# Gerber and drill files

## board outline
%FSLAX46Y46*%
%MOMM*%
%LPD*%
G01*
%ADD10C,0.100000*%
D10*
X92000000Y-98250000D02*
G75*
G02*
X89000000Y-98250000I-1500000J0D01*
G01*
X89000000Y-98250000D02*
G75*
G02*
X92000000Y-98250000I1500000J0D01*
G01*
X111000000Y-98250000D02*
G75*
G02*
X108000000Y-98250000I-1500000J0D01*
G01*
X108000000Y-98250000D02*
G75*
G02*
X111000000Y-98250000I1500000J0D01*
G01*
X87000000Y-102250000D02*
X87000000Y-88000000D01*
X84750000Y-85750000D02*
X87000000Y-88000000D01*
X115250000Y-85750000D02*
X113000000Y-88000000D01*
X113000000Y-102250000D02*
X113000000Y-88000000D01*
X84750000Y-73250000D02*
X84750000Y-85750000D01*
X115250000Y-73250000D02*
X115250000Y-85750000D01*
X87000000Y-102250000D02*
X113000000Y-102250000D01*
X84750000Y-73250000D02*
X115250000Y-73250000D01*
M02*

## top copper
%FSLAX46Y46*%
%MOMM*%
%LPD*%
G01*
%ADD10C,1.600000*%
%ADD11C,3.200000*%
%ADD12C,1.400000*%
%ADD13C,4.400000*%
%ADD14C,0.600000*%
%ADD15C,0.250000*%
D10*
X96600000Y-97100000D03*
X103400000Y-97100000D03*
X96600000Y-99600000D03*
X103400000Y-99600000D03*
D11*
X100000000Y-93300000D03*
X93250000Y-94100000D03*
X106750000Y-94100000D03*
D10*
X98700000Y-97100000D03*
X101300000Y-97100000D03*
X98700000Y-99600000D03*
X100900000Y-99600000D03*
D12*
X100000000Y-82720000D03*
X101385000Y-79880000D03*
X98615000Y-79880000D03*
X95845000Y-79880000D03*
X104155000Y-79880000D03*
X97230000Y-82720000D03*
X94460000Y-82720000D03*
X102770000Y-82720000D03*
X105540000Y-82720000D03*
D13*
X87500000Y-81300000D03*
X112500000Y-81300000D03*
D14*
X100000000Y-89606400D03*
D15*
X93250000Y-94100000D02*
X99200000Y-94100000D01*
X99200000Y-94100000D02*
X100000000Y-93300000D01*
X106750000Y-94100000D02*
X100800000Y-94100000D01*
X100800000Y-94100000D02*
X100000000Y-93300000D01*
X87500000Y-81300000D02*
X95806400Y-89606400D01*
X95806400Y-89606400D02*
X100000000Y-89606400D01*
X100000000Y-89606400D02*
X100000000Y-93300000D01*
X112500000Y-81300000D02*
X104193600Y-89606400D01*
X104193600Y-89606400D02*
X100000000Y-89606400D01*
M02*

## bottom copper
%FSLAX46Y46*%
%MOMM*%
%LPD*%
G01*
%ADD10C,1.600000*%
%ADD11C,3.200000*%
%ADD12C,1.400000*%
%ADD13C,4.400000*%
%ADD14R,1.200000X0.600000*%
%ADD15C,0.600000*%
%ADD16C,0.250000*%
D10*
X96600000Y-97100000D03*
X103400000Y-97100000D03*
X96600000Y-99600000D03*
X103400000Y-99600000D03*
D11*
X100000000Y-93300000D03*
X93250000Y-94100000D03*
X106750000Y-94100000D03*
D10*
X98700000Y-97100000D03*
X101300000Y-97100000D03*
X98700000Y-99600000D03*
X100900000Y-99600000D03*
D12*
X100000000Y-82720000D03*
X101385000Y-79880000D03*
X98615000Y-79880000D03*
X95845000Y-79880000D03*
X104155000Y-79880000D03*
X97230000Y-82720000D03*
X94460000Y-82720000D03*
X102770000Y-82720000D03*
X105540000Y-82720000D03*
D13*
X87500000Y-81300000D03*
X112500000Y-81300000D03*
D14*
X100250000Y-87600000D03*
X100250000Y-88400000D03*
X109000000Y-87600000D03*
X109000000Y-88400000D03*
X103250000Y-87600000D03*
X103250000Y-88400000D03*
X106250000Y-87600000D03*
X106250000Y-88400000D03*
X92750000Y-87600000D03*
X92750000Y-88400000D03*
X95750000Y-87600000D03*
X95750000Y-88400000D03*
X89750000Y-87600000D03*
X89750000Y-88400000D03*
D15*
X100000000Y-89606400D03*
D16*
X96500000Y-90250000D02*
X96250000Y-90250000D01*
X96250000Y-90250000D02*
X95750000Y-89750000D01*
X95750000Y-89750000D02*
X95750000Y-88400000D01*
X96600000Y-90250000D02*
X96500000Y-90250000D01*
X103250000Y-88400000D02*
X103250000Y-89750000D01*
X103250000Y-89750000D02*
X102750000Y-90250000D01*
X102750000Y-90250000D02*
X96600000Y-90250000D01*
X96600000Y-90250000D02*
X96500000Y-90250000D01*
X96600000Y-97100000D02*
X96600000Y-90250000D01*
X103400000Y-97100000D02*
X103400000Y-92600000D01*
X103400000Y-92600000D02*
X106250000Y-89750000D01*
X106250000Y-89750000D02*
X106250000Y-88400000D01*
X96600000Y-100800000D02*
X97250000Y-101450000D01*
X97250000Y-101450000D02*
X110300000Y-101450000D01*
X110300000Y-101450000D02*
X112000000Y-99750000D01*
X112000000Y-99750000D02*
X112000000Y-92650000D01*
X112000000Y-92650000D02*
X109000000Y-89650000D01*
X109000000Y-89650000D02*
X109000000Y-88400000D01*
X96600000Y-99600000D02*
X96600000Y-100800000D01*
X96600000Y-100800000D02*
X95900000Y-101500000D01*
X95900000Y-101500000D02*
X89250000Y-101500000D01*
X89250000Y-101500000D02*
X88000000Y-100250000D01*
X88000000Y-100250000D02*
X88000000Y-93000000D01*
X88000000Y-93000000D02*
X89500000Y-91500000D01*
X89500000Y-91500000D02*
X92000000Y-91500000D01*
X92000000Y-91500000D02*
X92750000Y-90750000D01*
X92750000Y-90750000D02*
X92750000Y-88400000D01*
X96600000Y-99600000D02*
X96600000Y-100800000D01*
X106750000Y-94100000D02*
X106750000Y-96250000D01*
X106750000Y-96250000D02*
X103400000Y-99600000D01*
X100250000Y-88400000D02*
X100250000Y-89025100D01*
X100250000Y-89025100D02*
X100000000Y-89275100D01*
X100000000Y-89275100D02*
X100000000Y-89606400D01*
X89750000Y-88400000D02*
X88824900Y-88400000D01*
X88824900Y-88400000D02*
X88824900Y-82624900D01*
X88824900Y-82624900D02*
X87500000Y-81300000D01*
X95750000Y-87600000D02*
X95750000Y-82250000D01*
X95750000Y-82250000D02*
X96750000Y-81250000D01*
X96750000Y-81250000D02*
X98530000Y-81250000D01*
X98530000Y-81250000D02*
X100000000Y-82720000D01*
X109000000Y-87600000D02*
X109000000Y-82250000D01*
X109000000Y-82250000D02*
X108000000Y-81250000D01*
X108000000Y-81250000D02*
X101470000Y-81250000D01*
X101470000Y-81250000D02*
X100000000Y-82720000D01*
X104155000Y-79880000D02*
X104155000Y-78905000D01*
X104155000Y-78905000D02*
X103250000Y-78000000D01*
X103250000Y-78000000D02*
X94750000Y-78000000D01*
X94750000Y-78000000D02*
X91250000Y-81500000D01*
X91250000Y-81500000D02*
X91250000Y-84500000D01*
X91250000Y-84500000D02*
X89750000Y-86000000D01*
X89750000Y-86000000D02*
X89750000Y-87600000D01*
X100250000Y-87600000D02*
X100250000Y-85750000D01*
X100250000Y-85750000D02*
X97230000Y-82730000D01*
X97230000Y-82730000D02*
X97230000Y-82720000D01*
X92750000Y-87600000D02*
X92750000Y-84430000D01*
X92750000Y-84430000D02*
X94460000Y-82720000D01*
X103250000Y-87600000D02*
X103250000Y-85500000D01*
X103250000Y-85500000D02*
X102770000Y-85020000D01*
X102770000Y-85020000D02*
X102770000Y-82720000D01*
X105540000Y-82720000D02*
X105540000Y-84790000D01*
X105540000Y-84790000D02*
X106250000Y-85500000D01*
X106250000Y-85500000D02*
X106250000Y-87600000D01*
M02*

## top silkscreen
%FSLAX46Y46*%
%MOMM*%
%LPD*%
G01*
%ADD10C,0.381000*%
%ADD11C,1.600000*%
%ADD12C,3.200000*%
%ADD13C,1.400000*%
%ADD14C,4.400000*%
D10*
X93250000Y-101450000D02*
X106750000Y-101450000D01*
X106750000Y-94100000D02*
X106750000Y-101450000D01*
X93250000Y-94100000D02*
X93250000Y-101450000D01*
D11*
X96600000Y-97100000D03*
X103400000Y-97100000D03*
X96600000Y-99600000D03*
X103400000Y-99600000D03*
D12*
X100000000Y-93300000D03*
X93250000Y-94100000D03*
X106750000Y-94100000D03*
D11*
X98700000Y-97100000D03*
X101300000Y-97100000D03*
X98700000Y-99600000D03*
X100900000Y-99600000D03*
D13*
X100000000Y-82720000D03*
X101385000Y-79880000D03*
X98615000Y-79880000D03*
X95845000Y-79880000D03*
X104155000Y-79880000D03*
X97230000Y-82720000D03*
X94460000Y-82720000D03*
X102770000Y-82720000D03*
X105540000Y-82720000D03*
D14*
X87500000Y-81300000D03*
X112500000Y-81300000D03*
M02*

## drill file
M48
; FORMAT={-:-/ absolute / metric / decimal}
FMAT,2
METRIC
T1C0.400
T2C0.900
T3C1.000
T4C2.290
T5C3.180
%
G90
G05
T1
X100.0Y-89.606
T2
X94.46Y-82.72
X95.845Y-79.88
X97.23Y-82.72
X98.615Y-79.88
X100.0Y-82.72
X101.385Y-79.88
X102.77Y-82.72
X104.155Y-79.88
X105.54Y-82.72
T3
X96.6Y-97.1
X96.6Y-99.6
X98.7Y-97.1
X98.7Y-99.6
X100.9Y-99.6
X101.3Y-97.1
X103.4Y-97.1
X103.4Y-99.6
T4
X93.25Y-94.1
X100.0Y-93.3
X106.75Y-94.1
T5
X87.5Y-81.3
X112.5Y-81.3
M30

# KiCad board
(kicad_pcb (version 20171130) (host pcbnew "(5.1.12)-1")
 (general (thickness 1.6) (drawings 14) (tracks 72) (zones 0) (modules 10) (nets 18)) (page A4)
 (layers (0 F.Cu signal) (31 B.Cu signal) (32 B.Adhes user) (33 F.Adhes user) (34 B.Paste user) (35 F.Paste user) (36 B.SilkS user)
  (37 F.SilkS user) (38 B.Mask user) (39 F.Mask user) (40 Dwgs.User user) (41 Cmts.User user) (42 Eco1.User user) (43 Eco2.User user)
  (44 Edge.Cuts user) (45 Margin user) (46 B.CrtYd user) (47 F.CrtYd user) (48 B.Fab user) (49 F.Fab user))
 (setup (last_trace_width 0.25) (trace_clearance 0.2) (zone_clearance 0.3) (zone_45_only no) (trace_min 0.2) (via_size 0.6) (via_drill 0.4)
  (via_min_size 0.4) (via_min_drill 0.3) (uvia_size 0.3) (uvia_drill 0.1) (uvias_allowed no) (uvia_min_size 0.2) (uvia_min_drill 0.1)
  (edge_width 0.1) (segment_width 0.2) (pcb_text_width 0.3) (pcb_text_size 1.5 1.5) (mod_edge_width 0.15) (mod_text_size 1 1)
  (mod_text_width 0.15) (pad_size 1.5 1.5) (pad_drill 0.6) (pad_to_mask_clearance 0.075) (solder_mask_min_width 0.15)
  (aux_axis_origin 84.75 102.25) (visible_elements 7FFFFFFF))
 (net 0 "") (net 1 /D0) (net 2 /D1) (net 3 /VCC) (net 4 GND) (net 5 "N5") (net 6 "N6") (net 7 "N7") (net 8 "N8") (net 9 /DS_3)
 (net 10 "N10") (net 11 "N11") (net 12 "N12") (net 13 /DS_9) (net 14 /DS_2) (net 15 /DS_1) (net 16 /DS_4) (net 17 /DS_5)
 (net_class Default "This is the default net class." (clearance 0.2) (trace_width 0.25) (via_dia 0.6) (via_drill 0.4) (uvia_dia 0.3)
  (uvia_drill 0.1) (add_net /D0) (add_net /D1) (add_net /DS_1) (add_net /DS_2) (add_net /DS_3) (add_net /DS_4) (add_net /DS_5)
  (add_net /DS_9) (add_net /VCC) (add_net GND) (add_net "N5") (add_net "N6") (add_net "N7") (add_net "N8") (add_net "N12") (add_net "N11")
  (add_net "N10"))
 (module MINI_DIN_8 (layer F.Cu) (at 100 93.3)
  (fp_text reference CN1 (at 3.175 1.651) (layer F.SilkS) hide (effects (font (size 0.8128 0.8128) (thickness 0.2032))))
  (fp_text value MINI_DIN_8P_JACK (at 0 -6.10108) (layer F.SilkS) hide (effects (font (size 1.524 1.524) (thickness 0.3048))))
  (fp_line (start -6.75 8.15) (end 6.75 8.15) (layer F.SilkS) (width 0.381))
  (fp_line (start 6.75 0.8) (end 6.75 8.15) (layer F.SilkS) (width 0.381))
  (fp_line (start -6.75 0.8) (end -6.75 8.15) (layer F.SilkS) (width 0.381))
  (pad 3 thru_hole circle (at -3.4 3.8 180) (size 1.6 1.6) (drill 1) (layers *.Cu *.Mask F.SilkS) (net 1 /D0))
  (pad 5 thru_hole circle (at 3.4 3.8 180) (size 1.6 1.6) (drill 1) (layers *.Cu *.Mask F.SilkS) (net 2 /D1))
  (pad 6 thru_hole circle (at -3.4 6.3 180) (size 1.6 1.6) (drill 1) (layers *.Cu *.Mask F.SilkS) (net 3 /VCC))
  (pad 8 thru_hole circle (at 3.4 6.3 180) (size 1.6 1.6) (drill 1) (layers *.Cu *.Mask F.SilkS) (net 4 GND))
  (pad 9 thru_hole circle (at 0 0 180) (size 3.2 3.2) (drill 2.29) (layers *.Cu *.Mask F.SilkS) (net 4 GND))
  (pad 9 thru_hole circle (at -6.75 0.8 180) (size 3.2 3.2) (drill 2.29) (layers *.Cu *.Mask F.SilkS) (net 4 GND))
  (pad 9 thru_hole circle (at 6.75 0.8 180) (size 3.2 3.2) (drill 2.29) (layers *.Cu *.Mask F.SilkS) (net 4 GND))
  (pad 1 thru_hole circle (at -1.3 3.8 180) (size 1.6 1.6) (drill 1) (layers *.Cu *.Mask F.SilkS) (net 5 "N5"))
  (pad 2 thru_hole circle (at 1.3 3.8 180) (size 1.6 1.6) (drill 1) (layers *.Cu *.Mask F.SilkS) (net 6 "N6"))
  (pad 4 thru_hole circle (at -1.3 6.3 180) (size 1.6 1.6) (drill 1) (layers *.Cu *.Mask F.SilkS) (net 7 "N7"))
  (pad 7 thru_hole circle (at 0.9 6.3 180) (size 1.6 1.6) (drill 1) (layers *.Cu *.Mask F.SilkS) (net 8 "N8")))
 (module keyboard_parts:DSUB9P (layer F.Cu) (at 100 81.3 180)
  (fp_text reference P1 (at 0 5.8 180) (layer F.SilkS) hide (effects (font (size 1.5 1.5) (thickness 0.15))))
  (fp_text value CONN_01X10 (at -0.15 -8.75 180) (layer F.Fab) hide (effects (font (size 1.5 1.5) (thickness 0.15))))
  (pad 3 thru_hole circle (at 0 -1.42 180) (size 1.4 1.4) (drill 0.9) (layers *.Cu *.Mask F.SilkS) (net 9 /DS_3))
  (pad 8 thru_hole circle (at -1.385 1.42 180) (size 1.4 1.4) (drill 0.9) (layers *.Cu *.Mask F.SilkS) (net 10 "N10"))
  (pad 7 thru_hole circle (at 1.385 1.42 180) (size 1.4 1.4) (drill 0.9) (layers *.Cu *.Mask F.SilkS) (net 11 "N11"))
  (pad 6 thru_hole circle (at 4.155 1.42 180) (size 1.4 1.4) (drill 0.9) (layers *.Cu *.Mask F.SilkS) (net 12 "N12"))
  (pad 9 thru_hole circle (at -4.155 1.42 180) (size 1.4 1.4) (drill 0.9) (layers *.Cu *.Mask F.SilkS) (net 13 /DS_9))
  (pad 2 thru_hole circle (at 2.77 -1.42 180) (size 1.4 1.4) (drill 0.9) (layers *.Cu *.Mask F.SilkS) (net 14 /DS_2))
  (pad 1 thru_hole circle (at 5.54 -1.42 180) (size 1.4 1.4) (drill 0.9) (layers *.Cu *.Mask F.SilkS) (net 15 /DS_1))
  (pad 4 thru_hole circle (at -2.77 -1.42 180) (size 1.4 1.4) (drill 0.9) (layers *.Cu *.Mask F.SilkS) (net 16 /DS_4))
  (pad 5 thru_hole circle (at -5.54 -1.42 180) (size 1.4 1.4) (drill 0.9) (layers *.Cu *.Mask F.SilkS) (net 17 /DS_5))
  (pad 10 thru_hole circle (at 12.5 0 180) (size 4.4 4.4) (drill 3.18) (layers *.Cu *.Mask F.SilkS) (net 4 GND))
  (pad 10 thru_hole circle (at -12.5 0 180) (size 4.4 4.4) (drill 3.18) (layers *.Cu *.Mask F.SilkS) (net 4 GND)))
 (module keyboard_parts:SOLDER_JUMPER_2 (layer B.Cu) (at 100.25 88 90)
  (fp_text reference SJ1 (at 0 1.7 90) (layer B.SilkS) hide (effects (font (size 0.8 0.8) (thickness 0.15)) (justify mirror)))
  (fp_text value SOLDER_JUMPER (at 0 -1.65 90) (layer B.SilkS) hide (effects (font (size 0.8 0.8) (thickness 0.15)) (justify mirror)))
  (pad 2 smd rect (at 0.4 0 90) (size 0.6 1.2) (layers B.Cu B.Mask) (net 14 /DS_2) (clearance 0.1))
  (pad 1 smd rect (at -0.4 0 90) (size 0.6 1.2) (layers B.Cu B.Mask) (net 4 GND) (clearance 0.1)))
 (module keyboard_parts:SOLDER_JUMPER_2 (layer B.Cu) (at 109 88 90)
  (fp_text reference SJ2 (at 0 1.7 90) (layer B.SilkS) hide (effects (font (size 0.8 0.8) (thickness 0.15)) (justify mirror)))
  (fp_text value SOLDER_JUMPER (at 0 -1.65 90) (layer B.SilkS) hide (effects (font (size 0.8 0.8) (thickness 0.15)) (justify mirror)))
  (pad 2 smd rect (at 0.4 0 90) (size 0.6 1.2) (layers B.Cu B.Mask) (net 9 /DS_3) (clearance 0.1))
  (pad 1 smd rect (at -0.4 0 90) (size 0.6 1.2) (layers B.Cu B.Mask) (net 3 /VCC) (clearance 0.1)))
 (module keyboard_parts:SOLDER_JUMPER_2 (layer B.Cu) (at 103.25 88 90)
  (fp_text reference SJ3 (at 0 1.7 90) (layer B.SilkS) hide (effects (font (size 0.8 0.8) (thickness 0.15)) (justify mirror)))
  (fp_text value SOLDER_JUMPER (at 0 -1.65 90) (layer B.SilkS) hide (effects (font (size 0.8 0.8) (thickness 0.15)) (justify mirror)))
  (pad 2 smd rect (at 0.4 0 90) (size 0.6 1.2) (layers B.Cu B.Mask) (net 16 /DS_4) (clearance 0.1))
  (pad 1 smd rect (at -0.4 0 90) (size 0.6 1.2) (layers B.Cu B.Mask) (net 1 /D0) (clearance 0.1)))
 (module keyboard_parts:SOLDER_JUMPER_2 (layer B.Cu) (at 106.25 88 90)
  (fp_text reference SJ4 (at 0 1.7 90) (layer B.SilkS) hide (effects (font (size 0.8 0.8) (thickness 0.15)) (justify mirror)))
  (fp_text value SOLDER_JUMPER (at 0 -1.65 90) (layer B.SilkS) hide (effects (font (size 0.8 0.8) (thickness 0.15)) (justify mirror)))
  (pad 2 smd rect (at 0.4 0 90) (size 0.6 1.2) (layers B.Cu B.Mask) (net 17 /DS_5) (clearance 0.1))
  (pad 1 smd rect (at -0.4 0 90) (size 0.6 1.2) (layers B.Cu B.Mask) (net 2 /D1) (clearance 0.1)))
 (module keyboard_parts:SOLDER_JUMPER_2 (layer B.Cu) (at 92.75 88 90)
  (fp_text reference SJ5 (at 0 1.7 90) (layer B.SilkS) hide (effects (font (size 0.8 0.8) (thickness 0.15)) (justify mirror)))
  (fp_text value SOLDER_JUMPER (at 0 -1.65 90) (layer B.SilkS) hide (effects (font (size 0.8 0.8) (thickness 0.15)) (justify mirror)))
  (pad 2 smd rect (at 0.4 0 90) (size 0.6 1.2) (layers B.Cu B.Mask) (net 15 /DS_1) (clearance 0.1))
  (pad 1 smd rect (at -0.4 0 90) (size 0.6 1.2) (layers B.Cu B.Mask) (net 3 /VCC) (clearance 0.1)))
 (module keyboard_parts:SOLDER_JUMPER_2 (layer B.Cu) (at 95.75 88 90)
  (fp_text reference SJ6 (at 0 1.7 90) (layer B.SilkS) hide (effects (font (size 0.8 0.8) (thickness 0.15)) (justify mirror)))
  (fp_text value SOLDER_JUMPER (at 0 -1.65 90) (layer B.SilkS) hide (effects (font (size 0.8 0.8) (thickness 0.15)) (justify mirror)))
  (pad 2 smd rect (at 0.4 0 90) (size 0.6 1.2) (layers B.Cu B.Mask) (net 9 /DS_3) (clearance 0.1))
  (pad 1 smd rect (at -0.4 0 90) (size 0.6 1.2) (layers B.Cu B.Mask) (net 1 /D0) (clearance 0.1)))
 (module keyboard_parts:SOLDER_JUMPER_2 (layer B.Cu) (at 89.75 88 90)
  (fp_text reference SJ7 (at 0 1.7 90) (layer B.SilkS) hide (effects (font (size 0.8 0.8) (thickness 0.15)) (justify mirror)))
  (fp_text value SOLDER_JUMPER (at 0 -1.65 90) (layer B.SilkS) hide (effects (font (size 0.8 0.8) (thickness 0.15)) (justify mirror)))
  (pad 2 smd rect (at 0.4 0 90) (size 0.6 1.2) (layers B.Cu B.Mask) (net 13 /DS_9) (clearance 0.1))
  (pad 1 smd rect (at -0.4 0 90) (size 0.6 1.2) (layers B.Cu B.Mask) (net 4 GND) (clearance 0.1)))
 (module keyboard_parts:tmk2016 (layer B.Cu) (at 99.06 78.74 180)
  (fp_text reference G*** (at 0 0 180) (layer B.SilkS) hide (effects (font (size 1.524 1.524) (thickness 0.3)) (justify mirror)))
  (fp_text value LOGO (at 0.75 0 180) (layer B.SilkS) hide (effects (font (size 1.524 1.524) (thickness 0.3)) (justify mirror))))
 (gr_circle (center 90.5 98.25) (end 90.5 99.75) (layer Edge.Cuts) (width 0.1))
 (gr_circle (center 109.5 98.25) (end 109.5 99.75) (layer Edge.Cuts) (width 0.1))
 (gr_line (start 87 102.25) (end 87 88) (angle 90) (layer Edge.Cuts) (width 0.1))
 (gr_line (start 84.75 85.75) (end 87 88) (angle 90) (layer Edge.Cuts) (width 0.1))
 (gr_line (start 115.25 85.75) (end 113 88) (angle 90) (layer Edge.Cuts) (width 0.1))
 (gr_line (start 113 102.25) (end 113 88) (angle 90) (layer Edge.Cuts) (width 0.1))
 (gr_line (start 84.75 73.25) (end 84.75 85.75) (angle 90) (layer Edge.Cuts) (width 0.1))
 (gr_line (start 115.25 73.25) (end 115.25 85.75) (angle 90) (layer Edge.Cuts) (width 0.1))
 (gr_line (start 87 102.25) (end 113 102.25) (angle 90) (layer Edge.Cuts) (width 0.1))
 (gr_line (start 84.75 73.25) (end 115.25 73.25) (angle 90) (layer Edge.Cuts) (width 0.1))
 (segment (start 96.5 90.25) (end 96.25 90.25) (width 0.25) (layer B.Cu) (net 1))
 (segment (start 96.25 90.25) (end 95.75 89.75) (width 0.25) (layer B.Cu) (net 1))
 (segment (start 95.75 89.75) (end 95.75 88.4) (width 0.25) (layer B.Cu) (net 1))
 (segment (start 96.6 90.25) (end 96.5 90.25) (width 0.25) (layer B.Cu) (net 1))
 (segment (start 103.25 88.4) (end 103.25 89.75) (width 0.25) (layer B.Cu) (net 1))
 (segment (start 103.25 89.75) (end 102.75 90.25) (width 0.25) (layer B.Cu) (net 1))
 (segment (start 102.75 90.25) (end 96.6 90.25) (width 0.25) (layer B.Cu) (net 1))
 (segment (start 96.6 90.25) (end 96.5 90.25) (width 0.25) (layer B.Cu) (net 1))
 (segment (start 96.6 97.1) (end 96.6 90.25) (width 0.25) (layer B.Cu) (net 1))
 (segment (start 103.4 97.1) (end 103.4 92.6) (width 0.25) (layer B.Cu) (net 2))
 (segment (start 103.4 92.6) (end 106.25 89.75) (width 0.25) (layer B.Cu) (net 2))
 (segment (start 106.25 89.75) (end 106.25 88.4) (width 0.25) (layer B.Cu) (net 2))
 (segment (start 96.6 100.8) (end 97.25 101.45) (width 0.25) (layer B.Cu) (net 3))
 (segment (start 97.25 101.45) (end 110.3 101.45) (width 0.25) (layer B.Cu) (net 3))
 (segment (start 110.3 101.45) (end 112 99.75) (width 0.25) (layer B.Cu) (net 3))
 (segment (start 112 99.75) (end 112 92.65) (width 0.25) (layer B.Cu) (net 3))
 (segment (start 112 92.65) (end 109 89.65) (width 0.25) (layer B.Cu) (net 3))
 (segment (start 109 89.65) (end 109 88.4) (width 0.25) (layer B.Cu) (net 3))
 (segment (start 96.6 99.6) (end 96.6 100.8) (width 0.25) (layer B.Cu) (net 3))
 (segment (start 96.6 100.8) (end 95.9 101.5) (width 0.25) (layer B.Cu) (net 3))
 (segment (start 95.9 101.5) (end 89.25 101.5) (width 0.25) (layer B.Cu) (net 3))
 (segment (start 89.25 101.5) (end 88 100.25) (width 0.25) (layer B.Cu) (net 3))
 (segment (start 88 100.25) (end 88 93) (width 0.25) (layer B.Cu) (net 3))
 (segment (start 88 93) (end 89.5 91.5) (width 0.25) (layer B.Cu) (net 3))
 (segment (start 89.5 91.5) (end 92 91.5) (width 0.25) (layer B.Cu) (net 3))
 (segment (start 92 91.5) (end 92.75 90.75) (width 0.25) (layer B.Cu) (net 3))
 (segment (start 92.75 90.75) (end 92.75 88.4) (width 0.25) (layer B.Cu) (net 3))
 (segment (start 96.6 99.6) (end 96.6 100.8) (width 0.25) (layer B.Cu) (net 3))
 (segment (start 106.75 94.1) (end 106.75 96.25) (width 0.25) (layer B.Cu) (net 4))
 (segment (start 106.75 96.25) (end 103.4 99.6) (width 0.25) (layer B.Cu) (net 4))
 (segment (start 93.25 94.1) (end 99.2 94.1) (width 0.25) (layer F.Cu) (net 4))
 (segment (start 99.2 94.1) (end 100 93.3) (width 0.25) (layer F.Cu) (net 4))
 (segment (start 106.75 94.1) (end 100.8 94.1) (width 0.25) (layer F.Cu) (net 4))
 (segment (start 100.8 94.1) (end 100 93.3) (width 0.25) (layer F.Cu) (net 4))
 (segment (start 87.5 81.3) (end 95.8064 89.6064) (width 0.25) (layer F.Cu) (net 4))
 (segment (start 95.8064 89.6064) (end 100 89.6064) (width 0.25) (layer F.Cu) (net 4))
 (segment (start 100 89.6064) (end 100 93.3) (width 0.25) (layer F.Cu) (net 4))
 (segment (start 112.5 81.3) (end 104.1936 89.6064) (width 0.25) (layer F.Cu) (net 4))
 (segment (start 104.1936 89.6064) (end 100 89.6064) (width 0.25) (layer F.Cu) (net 4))
 (segment (start 100.25 88.4) (end 100.25 89.0251) (width 0.25) (layer B.Cu) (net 4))
 (segment (start 100.25 89.0251) (end 100 89.2751) (width 0.25) (layer B.Cu) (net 4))
 (segment (start 100 89.2751) (end 100 89.6064) (width 0.25) (layer B.Cu) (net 4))
 (segment (start 89.75 88.4) (end 88.8249 88.4) (width 0.25) (layer B.Cu) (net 4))
 (segment (start 88.8249 88.4) (end 88.8249 82.6249) (width 0.25) (layer B.Cu) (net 4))
 (segment (start 88.8249 82.6249) (end 87.5 81.3) (width 0.25) (layer B.Cu) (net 4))
 (via (at 100 89.6064) (size 0.6) (layers F.Cu B.Cu) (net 4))
 (segment (start 95.75 87.6) (end 95.75 82.25) (width 0.25) (layer B.Cu) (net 9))
 (segment (start 95.75 82.25) (end 96.75 81.25) (width 0.25) (layer B.Cu) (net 9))
 (segment (start 96.75 81.25) (end 98.53 81.25) (width 0.25) (layer B.Cu) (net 9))
 (segment (start 98.53 81.25) (end 100 82.72) (width 0.25) (layer B.Cu) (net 9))
 (segment (start 109 87.6) (end 109 82.25) (width 0.25) (layer B.Cu) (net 9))
 (segment (start 109 82.25) (end 108 81.25) (width 0.25) (layer B.Cu) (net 9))
 (segment (start 108 81.25) (end 101.47 81.25) (width 0.25) (layer B.Cu) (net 9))
 (segment (start 101.47 81.25) (end 100 82.72) (width 0.25) (layer B.Cu) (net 9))
 (segment (start 104.155 79.88) (end 104.155 78.905) (width 0.25) (layer B.Cu) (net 13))
 (segment (start 104.155 78.905) (end 103.25 78) (width 0.25) (layer B.Cu) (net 13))
 (segment (start 103.25 78) (end 94.75 78) (width 0.25) (layer B.Cu) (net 13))
 (segment (start 94.75 78) (end 91.25 81.5) (width 0.25) (layer B.Cu) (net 13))
 (segment (start 91.25 81.5) (end 91.25 84.5) (width 0.25) (layer B.Cu) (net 13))
 (segment (start 91.25 84.5) (end 89.75 86) (width 0.25) (layer B.Cu) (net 13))
 (segment (start 89.75 86) (end 89.75 87.6) (width 0.25) (layer B.Cu) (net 13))
 (segment (start 100.25 87.6) (end 100.25 85.75) (width 0.25) (layer B.Cu) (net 14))
 (segment (start 100.25 85.75) (end 97.23 82.73) (width 0.25) (layer B.Cu) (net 14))
 (segment (start 97.23 82.73) (end 97.23 82.72) (width 0.25) (layer B.Cu) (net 14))
 (segment (start 92.75 87.6) (end 92.75 84.43) (width 0.25) (layer B.Cu) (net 15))
 (segment (start 92.75 84.43) (end 94.46 82.72) (width 0.25) (layer B.Cu) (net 15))
 (segment (start 103.25 87.6) (end 103.25 85.5) (width 0.25) (layer B.Cu) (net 16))
 (segment (start 103.25 85.5) (end 102.77 85.02) (width 0.25) (layer B.Cu) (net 16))
 (segment (start 102.77 85.02) (end 102.77 82.72) (width 0.25) (layer B.Cu) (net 16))
 (segment (start 105.54 82.72) (end 105.54 84.79) (width 0.25) (layer B.Cu) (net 17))
 (segment (start 105.54 84.79) (end 106.25 85.5) (width 0.25) (layer B.Cu) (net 17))
 (segment (start 106.25 85.5) (end 106.25 87.6) (width 0.25) (layer B.Cu) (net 17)))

